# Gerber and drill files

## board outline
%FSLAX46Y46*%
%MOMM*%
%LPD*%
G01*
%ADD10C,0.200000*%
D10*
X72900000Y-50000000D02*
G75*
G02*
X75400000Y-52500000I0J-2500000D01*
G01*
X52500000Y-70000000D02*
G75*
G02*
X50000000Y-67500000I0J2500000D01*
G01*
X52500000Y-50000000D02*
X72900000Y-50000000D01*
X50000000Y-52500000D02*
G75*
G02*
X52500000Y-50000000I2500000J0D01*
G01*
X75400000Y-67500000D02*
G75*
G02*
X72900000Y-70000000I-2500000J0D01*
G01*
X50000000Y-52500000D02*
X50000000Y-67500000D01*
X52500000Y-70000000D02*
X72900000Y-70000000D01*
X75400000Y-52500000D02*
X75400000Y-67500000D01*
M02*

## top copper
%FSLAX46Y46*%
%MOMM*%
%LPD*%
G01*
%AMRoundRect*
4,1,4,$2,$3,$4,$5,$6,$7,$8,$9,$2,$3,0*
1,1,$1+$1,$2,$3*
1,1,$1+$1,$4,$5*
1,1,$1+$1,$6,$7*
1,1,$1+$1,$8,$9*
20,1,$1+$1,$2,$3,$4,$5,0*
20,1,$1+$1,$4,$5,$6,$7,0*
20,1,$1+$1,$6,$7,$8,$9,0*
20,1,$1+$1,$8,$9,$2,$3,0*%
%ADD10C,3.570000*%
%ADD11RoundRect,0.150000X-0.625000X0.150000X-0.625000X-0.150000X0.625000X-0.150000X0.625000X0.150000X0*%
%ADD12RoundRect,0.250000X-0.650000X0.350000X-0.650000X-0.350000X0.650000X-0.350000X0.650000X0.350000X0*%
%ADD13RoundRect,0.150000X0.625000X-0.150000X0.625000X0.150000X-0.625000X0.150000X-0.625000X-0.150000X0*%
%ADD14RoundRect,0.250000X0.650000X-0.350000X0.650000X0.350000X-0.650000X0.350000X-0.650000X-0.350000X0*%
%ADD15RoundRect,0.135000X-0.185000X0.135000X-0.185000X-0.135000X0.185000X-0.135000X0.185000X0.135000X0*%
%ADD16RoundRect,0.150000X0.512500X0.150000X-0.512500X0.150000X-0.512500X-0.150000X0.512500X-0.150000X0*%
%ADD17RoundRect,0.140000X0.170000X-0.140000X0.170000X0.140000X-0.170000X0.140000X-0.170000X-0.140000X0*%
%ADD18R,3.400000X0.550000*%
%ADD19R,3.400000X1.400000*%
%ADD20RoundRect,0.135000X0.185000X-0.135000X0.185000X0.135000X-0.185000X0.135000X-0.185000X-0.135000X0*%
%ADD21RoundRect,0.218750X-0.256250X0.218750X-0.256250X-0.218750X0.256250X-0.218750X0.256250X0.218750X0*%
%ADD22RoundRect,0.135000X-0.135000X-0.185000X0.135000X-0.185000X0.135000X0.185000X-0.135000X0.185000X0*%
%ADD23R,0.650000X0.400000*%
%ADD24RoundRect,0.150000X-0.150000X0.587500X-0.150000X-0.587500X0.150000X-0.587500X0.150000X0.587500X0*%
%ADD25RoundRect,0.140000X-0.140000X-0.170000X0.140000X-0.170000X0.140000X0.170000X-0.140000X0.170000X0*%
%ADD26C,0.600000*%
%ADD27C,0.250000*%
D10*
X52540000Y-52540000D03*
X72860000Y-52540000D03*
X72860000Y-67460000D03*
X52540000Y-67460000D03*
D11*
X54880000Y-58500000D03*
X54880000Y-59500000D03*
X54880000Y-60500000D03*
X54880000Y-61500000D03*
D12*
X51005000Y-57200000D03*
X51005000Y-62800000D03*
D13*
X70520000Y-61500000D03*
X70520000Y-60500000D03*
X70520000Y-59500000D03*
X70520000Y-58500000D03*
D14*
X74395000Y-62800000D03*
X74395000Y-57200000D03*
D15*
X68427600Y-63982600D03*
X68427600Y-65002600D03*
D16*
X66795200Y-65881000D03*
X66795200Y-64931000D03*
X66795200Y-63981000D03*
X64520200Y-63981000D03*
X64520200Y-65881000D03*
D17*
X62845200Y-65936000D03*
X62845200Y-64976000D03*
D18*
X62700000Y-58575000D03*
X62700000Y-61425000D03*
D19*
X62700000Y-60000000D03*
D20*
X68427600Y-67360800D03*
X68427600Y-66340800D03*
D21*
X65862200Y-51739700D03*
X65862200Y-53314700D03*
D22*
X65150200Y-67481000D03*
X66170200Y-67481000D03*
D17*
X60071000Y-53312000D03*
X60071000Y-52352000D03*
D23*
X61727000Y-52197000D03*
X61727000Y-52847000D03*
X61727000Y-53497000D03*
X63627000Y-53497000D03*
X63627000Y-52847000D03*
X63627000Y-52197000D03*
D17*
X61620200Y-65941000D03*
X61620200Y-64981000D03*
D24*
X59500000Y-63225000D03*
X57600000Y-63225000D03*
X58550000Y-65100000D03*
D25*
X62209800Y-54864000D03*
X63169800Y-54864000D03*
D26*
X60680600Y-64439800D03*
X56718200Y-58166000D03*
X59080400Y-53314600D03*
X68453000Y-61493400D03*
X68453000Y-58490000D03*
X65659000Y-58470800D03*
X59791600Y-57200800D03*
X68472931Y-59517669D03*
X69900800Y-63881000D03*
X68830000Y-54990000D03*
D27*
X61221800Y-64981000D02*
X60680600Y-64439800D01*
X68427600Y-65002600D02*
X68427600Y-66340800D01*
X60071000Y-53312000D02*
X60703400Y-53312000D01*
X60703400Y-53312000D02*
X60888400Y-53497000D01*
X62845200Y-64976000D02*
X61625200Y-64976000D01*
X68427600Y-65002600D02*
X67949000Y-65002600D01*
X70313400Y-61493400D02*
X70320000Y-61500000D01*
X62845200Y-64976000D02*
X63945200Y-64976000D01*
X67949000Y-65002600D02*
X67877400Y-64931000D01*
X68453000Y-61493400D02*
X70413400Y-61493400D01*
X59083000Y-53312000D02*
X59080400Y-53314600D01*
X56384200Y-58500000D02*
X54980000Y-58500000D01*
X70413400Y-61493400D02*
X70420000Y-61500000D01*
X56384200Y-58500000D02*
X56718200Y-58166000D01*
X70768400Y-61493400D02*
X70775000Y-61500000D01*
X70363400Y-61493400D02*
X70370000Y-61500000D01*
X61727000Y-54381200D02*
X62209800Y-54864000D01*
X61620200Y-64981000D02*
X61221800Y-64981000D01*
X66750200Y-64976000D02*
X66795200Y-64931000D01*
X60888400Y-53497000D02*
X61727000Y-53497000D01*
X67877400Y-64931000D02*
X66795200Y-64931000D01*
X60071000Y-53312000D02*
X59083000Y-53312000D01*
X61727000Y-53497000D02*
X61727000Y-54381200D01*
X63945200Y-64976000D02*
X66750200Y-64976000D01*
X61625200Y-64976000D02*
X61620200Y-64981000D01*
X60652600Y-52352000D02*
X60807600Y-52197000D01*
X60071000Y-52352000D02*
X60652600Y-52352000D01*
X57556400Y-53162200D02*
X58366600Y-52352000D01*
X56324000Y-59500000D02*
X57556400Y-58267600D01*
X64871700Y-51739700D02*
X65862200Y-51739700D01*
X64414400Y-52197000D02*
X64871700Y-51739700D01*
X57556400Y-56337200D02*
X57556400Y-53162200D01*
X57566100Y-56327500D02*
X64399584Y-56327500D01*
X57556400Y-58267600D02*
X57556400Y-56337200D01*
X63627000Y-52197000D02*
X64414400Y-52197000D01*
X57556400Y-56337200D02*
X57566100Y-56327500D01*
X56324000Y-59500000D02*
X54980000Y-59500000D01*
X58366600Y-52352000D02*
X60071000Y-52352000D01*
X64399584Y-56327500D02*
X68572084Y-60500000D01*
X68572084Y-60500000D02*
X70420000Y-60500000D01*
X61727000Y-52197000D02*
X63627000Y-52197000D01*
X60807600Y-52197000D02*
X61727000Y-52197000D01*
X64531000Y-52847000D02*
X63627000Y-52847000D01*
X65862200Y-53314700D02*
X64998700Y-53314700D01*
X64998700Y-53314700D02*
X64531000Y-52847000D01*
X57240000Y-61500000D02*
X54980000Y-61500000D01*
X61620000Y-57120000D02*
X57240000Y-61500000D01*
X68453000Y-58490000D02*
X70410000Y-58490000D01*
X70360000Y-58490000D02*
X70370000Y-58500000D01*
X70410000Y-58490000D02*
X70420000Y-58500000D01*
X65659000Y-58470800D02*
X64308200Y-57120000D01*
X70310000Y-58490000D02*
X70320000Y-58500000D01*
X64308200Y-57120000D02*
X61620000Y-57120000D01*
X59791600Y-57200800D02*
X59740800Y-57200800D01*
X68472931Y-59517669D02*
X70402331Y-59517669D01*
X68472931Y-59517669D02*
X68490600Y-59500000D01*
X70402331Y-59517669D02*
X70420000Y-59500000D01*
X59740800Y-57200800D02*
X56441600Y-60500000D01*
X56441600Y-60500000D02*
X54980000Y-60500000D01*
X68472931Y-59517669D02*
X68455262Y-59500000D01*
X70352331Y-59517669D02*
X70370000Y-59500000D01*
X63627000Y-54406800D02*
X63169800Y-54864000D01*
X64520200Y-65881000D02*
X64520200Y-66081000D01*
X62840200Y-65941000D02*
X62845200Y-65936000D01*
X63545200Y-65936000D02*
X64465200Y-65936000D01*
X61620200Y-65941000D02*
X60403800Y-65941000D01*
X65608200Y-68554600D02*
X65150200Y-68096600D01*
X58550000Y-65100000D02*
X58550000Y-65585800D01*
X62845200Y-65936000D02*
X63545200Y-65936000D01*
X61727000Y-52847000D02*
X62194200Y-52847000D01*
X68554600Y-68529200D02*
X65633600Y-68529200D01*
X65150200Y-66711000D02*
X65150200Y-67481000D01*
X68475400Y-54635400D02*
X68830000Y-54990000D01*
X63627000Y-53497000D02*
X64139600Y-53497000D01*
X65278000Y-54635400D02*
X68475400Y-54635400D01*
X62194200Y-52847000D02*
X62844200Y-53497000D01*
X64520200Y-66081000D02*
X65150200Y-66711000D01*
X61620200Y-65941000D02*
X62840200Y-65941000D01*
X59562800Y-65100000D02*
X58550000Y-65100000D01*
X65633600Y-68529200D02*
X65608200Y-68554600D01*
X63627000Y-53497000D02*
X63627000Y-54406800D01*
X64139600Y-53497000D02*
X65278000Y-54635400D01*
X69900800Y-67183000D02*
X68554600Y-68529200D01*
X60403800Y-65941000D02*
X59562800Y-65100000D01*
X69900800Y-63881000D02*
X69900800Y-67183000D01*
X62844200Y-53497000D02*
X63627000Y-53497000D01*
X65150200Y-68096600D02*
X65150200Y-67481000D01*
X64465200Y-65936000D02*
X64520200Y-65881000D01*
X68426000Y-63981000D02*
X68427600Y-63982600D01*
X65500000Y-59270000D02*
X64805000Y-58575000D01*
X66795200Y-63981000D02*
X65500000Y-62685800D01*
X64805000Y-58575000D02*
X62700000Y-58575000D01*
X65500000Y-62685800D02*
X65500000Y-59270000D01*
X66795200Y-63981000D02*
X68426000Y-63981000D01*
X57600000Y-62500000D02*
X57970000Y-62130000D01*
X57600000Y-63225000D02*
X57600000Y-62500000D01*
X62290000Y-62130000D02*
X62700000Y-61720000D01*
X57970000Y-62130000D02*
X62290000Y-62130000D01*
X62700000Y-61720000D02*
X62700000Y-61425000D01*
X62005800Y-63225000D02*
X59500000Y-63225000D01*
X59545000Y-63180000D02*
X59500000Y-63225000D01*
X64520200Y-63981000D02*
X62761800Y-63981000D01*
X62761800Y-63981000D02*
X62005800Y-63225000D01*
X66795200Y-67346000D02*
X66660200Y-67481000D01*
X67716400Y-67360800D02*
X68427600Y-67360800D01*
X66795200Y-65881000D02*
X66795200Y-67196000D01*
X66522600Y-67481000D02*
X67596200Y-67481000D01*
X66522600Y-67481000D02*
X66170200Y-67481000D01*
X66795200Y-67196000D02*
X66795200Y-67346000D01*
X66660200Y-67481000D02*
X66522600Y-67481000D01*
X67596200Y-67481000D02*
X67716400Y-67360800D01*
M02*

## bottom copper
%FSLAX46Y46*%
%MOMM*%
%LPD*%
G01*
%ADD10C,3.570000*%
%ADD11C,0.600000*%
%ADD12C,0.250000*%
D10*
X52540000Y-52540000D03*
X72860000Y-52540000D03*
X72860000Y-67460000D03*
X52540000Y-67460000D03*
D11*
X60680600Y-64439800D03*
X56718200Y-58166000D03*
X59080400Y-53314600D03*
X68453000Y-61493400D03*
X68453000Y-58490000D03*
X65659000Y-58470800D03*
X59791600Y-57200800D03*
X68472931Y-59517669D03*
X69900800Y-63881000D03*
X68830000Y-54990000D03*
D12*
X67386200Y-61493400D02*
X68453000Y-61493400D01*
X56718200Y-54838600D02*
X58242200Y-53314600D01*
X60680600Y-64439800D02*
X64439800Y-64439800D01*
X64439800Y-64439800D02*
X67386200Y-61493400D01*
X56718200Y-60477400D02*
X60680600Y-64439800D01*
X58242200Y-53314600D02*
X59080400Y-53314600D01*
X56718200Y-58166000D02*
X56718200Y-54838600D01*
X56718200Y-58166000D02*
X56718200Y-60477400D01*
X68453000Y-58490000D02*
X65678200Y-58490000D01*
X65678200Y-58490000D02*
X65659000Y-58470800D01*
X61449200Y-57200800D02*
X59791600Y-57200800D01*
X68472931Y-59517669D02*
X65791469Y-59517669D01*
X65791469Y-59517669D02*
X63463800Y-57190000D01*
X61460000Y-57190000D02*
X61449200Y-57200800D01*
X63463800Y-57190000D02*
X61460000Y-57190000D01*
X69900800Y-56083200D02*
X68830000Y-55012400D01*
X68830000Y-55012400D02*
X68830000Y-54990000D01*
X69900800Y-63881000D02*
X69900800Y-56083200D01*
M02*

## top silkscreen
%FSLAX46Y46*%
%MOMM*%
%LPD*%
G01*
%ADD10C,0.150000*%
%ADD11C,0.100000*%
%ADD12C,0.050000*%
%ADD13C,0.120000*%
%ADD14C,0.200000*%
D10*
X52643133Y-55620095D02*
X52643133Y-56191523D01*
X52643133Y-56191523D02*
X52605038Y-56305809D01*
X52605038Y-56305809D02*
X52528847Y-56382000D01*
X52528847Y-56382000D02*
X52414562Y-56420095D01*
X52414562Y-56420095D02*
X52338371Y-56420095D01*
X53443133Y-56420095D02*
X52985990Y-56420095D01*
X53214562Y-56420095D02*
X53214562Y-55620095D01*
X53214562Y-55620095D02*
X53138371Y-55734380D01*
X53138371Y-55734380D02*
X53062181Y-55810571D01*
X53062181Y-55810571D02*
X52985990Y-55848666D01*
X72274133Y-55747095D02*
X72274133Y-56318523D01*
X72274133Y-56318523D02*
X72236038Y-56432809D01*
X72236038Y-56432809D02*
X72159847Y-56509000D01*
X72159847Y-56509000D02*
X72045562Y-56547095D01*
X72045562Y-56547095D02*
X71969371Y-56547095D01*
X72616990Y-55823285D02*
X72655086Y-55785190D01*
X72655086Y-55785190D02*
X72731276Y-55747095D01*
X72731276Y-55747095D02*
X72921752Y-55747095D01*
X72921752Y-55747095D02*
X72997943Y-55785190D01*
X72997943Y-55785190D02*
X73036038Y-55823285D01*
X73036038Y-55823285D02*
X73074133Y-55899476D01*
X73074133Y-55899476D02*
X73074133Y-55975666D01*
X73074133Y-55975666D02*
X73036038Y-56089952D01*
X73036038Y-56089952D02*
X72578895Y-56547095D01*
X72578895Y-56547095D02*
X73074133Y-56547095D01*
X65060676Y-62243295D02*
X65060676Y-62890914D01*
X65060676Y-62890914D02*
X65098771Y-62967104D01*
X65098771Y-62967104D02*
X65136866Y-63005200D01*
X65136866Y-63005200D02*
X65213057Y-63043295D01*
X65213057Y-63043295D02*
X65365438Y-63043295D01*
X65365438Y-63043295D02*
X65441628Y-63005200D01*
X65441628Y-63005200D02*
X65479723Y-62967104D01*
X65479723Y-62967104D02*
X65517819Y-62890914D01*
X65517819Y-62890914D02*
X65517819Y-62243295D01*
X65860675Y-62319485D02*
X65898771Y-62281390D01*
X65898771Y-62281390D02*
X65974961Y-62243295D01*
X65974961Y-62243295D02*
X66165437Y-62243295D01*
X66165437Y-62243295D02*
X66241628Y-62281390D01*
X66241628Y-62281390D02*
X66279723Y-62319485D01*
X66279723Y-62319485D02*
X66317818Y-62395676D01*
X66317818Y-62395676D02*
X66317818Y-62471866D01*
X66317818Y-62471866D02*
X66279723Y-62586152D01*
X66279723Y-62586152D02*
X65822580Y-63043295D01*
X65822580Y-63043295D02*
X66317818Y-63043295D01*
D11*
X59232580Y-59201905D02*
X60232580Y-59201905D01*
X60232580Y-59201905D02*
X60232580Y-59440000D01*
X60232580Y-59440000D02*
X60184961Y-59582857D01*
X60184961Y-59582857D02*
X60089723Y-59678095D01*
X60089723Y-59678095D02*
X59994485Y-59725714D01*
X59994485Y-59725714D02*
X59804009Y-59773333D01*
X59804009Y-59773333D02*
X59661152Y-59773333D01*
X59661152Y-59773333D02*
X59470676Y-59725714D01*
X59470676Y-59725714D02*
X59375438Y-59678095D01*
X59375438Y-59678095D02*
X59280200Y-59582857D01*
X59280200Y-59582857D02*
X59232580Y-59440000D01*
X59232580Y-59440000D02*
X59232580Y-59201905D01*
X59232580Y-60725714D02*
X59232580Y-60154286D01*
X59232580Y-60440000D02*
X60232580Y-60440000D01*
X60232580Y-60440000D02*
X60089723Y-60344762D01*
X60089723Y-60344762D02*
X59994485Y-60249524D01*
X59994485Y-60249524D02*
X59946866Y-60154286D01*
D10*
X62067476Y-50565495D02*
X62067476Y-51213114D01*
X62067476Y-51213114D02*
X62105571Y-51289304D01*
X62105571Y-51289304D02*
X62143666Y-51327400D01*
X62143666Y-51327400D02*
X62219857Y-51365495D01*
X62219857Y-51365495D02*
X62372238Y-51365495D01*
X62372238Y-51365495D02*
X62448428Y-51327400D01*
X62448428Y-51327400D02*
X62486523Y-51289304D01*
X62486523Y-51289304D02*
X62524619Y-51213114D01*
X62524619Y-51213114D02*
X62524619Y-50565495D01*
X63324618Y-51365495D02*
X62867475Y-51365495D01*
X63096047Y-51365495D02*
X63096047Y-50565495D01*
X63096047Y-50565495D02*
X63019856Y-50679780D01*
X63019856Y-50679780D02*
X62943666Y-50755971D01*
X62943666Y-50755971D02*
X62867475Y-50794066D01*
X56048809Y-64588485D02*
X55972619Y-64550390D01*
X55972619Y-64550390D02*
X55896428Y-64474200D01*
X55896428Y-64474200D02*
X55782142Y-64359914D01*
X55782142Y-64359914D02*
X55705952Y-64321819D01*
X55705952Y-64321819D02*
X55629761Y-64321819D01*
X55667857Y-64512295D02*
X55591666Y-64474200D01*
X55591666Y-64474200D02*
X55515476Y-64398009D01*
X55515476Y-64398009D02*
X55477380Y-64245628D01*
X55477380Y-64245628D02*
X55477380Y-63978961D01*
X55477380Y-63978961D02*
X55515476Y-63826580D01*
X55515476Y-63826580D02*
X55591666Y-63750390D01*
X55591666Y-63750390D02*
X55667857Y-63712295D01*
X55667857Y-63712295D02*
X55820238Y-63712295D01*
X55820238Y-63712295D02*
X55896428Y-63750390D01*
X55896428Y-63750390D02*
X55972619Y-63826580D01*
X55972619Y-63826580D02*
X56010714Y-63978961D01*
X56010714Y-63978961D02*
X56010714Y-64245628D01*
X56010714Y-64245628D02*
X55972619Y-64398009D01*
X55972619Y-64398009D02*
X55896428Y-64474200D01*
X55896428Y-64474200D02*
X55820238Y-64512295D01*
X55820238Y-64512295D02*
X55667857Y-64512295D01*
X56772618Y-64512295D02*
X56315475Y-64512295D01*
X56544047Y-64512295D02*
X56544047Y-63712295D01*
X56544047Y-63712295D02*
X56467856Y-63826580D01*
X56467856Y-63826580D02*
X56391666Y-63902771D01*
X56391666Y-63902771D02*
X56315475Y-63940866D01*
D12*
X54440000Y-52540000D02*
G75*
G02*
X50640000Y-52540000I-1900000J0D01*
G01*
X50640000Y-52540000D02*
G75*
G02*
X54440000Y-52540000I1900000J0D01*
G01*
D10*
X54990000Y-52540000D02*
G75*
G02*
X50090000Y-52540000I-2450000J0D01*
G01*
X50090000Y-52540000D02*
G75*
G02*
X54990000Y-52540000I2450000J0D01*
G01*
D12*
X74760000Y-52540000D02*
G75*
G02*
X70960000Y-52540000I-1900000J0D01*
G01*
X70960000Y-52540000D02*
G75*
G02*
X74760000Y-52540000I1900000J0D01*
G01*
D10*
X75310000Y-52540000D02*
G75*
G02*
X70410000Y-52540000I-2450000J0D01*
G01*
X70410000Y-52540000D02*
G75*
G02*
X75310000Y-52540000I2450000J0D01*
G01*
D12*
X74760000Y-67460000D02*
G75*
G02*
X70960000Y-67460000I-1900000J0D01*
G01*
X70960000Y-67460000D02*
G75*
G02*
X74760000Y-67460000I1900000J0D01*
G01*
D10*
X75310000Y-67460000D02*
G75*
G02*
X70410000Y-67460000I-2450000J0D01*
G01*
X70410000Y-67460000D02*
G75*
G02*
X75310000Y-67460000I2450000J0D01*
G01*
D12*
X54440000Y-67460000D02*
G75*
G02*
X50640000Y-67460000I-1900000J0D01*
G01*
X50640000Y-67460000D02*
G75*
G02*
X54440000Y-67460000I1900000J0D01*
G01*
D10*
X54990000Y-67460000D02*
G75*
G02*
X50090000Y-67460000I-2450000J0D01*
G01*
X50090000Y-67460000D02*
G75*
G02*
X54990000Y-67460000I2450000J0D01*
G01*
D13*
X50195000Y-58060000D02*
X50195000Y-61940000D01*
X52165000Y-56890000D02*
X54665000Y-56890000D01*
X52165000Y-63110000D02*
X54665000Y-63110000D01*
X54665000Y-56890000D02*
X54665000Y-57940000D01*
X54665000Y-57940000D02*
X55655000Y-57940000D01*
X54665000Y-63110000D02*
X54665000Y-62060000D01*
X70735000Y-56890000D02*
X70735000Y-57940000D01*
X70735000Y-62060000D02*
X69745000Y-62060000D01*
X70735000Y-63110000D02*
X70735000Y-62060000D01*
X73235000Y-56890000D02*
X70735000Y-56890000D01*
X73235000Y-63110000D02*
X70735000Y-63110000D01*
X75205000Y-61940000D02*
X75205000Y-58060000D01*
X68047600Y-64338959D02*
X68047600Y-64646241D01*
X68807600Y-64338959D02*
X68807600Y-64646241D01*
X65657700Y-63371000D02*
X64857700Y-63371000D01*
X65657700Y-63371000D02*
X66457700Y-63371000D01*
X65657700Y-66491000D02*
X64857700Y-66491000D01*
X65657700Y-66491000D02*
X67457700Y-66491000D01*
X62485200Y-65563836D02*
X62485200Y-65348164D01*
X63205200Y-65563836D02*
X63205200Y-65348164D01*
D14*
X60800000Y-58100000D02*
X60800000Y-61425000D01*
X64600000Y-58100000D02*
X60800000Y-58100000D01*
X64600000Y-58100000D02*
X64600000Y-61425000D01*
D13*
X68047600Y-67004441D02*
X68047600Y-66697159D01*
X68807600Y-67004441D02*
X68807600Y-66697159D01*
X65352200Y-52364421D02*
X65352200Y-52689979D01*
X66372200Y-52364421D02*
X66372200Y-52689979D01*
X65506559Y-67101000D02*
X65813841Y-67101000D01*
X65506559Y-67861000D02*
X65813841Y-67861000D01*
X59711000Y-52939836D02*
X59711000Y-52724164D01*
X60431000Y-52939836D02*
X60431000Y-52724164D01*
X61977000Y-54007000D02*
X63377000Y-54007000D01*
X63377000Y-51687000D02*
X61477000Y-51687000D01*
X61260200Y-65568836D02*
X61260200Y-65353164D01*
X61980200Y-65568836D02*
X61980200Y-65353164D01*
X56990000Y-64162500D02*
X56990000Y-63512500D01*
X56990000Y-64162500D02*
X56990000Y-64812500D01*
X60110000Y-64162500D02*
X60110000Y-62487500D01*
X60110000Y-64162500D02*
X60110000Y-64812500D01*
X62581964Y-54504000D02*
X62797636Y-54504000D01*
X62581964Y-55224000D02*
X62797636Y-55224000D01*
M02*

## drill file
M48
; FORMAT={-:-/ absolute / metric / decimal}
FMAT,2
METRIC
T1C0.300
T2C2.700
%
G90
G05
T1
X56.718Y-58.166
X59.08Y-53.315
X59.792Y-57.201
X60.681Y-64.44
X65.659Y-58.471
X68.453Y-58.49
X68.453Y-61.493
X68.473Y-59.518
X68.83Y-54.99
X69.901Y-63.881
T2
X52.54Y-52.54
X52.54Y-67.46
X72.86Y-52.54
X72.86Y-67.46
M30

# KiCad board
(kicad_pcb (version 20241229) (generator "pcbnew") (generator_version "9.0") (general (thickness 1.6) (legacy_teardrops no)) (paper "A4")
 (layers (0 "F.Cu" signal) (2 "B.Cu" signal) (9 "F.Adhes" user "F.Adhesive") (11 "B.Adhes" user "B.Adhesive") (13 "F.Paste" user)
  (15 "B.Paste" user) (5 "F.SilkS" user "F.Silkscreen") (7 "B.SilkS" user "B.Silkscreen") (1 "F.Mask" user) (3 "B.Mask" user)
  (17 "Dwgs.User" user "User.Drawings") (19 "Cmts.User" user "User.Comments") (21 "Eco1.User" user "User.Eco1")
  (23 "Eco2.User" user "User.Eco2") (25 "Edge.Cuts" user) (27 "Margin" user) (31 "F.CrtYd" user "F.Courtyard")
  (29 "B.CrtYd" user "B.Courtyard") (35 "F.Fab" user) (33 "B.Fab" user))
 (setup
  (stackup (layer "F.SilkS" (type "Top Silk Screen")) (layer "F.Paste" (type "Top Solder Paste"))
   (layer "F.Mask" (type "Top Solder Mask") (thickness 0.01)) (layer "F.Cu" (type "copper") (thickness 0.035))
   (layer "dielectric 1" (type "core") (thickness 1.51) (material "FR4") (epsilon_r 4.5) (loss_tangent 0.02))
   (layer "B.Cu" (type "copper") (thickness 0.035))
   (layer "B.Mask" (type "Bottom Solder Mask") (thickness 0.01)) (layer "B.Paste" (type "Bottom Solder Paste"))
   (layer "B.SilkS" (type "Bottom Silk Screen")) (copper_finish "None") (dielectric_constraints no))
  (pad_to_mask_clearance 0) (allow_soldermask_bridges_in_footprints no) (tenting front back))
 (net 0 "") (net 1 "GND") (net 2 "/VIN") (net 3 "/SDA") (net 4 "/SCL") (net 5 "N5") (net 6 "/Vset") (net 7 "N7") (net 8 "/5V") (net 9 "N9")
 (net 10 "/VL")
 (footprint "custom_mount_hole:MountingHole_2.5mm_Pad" (layer "F.Cu") (at 52.54 52.54)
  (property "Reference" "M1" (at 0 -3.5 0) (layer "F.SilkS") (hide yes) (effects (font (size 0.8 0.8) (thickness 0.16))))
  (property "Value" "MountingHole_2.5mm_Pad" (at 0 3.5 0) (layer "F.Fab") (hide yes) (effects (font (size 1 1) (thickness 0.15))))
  (fp_circle (center 0 0) (end 1.9 0) (stroke (width 0.05) (type solid)) (fill no) (layer "F.SilkS"))
  (fp_circle (center 0 0) (end 2.45 0) (stroke (width 0.15) (type solid)) (fill no) (layer "F.SilkS"))
  (pad "~" thru_hole circle (at 0 0) (size 3.57 3.57) (drill 2.7) (layers "*.Cu" "*.Mask") (remove_unused_layers no)))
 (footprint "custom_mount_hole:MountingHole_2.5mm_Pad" (layer "F.Cu") (at 72.86 52.54)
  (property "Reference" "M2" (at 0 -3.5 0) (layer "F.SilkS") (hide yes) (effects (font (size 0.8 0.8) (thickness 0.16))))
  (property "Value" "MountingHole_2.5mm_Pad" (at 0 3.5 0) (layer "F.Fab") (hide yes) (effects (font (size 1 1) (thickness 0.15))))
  (fp_circle (center 0 0) (end 1.9 0) (stroke (width 0.05) (type solid)) (fill no) (layer "F.SilkS"))
  (fp_circle (center 0 0) (end 2.45 0) (stroke (width 0.15) (type solid)) (fill no) (layer "F.SilkS"))
  (pad "~" thru_hole circle (at 0 0) (size 3.57 3.57) (drill 2.7) (layers "*.Cu" "*.Mask") (remove_unused_layers no)))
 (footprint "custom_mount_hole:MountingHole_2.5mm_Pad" (layer "F.Cu") (at 72.86 67.46)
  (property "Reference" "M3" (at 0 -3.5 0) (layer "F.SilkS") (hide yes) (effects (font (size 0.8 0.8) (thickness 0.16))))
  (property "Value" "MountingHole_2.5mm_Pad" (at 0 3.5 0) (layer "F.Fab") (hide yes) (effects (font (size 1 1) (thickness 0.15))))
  (fp_circle (center 0 0) (end 1.9 0) (stroke (width 0.05) (type solid)) (fill no) (layer "F.SilkS"))
  (fp_circle (center 0 0) (end 2.45 0) (stroke (width 0.15) (type solid)) (fill no) (layer "F.SilkS"))
  (pad "~" thru_hole circle (at 0 0) (size 3.57 3.57) (drill 2.7) (layers "*.Cu" "*.Mask") (remove_unused_layers no)))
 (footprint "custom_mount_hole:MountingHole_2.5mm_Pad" (layer "F.Cu") (at 52.54 67.46)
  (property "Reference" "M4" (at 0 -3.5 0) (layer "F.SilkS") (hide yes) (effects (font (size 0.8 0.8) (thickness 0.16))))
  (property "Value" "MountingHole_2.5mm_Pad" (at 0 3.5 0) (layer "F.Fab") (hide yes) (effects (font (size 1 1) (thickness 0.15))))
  (fp_circle (center 0 0) (end 1.9 0) (stroke (width 0.05) (type solid)) (fill no) (layer "F.SilkS"))
  (fp_circle (center 0 0) (end 2.45 0) (stroke (width 0.15) (type solid)) (fill no) (layer "F.SilkS"))
  (pad "~" thru_hole circle (at 0 0) (size 3.57 3.57) (drill 2.7) (layers "*.Cu" "*.Mask") (remove_unused_layers no)))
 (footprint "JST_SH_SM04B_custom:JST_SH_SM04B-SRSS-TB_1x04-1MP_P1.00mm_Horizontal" (layer "F.Cu") (at 52.88 60 -90)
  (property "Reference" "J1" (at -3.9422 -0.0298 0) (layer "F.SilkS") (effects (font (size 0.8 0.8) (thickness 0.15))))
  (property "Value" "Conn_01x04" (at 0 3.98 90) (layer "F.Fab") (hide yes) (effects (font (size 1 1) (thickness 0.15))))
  (fp_line (start -1.94 2.685) (end 1.94 2.685) (stroke (width 0.12) (type solid)) (layer "F.SilkS"))
  (fp_line (start -3.11 0.715) (end -3.11 -1.785) (stroke (width 0.12) (type solid)) (layer "F.SilkS"))
  (fp_line (start 3.11 0.715) (end 3.11 -1.785) (stroke (width 0.12) (type solid)) (layer "F.SilkS"))
  (fp_line (start -3.11 -1.785) (end -2.06 -1.785) (stroke (width 0.12) (type solid)) (layer "F.SilkS"))
  (fp_line (start -2.06 -1.785) (end -2.06 -2.775) (stroke (width 0.12) (type solid)) (layer "F.SilkS"))
  (fp_line (start 3.11 -1.785) (end 2.06 -1.785) (stroke (width 0.12) (type solid)) (layer "F.SilkS"))
  (pad "1" smd roundrect (at -1.5 -2 270) (size 0.6 1.55) (layers "F.Cu" "F.Mask" "F.Paste") (roundrect_rratio 0.25) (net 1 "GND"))
  (pad "2" smd roundrect (at -0.5 -2 270) (size 0.6 1.55) (layers "F.Cu" "F.Mask" "F.Paste") (roundrect_rratio 0.25) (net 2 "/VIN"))
  (pad "3" smd roundrect (at 0.5 -2 270) (size 0.6 1.55) (layers "F.Cu" "F.Mask" "F.Paste") (roundrect_rratio 0.25) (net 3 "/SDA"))
  (pad "4" smd roundrect (at 1.5 -2 270) (size 0.6 1.55) (layers "F.Cu" "F.Mask" "F.Paste") (roundrect_rratio 0.25) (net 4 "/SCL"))
  (pad "MP" smd roundrect (at -2.8 1.875 270) (size 1.2 1.8) (layers "F.Cu" "F.Mask" "F.Paste") (roundrect_rratio 0.2083333333))
  (pad "MP" smd roundrect (at 2.8 1.875 270) (size 1.2 1.8) (layers "F.Cu" "F.Mask" "F.Paste") (roundrect_rratio 0.2083333333)))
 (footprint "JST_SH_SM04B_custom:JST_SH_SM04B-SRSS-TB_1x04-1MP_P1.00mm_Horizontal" (layer "F.Cu") (at 72.52 60 90)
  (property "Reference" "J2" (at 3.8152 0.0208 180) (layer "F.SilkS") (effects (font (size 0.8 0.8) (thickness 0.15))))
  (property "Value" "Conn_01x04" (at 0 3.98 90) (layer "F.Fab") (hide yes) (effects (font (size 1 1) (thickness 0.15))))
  (fp_line (start 3.11 -1.785) (end 2.06 -1.785) (stroke (width 0.12) (type solid)) (layer "F.SilkS"))
  (fp_line (start -2.06 -1.785) (end -2.06 -2.775) (stroke (width 0.12) (type solid)) (layer "F.SilkS"))
  (fp_line (start -3.11 -1.785) (end -2.06 -1.785) (stroke (width 0.12) (type solid)) (layer "F.SilkS"))
  (fp_line (start 3.11 0.715) (end 3.11 -1.785) (stroke (width 0.12) (type solid)) (layer "F.SilkS"))
  (fp_line (start -3.11 0.715) (end -3.11 -1.785) (stroke (width 0.12) (type solid)) (layer "F.SilkS"))
  (fp_line (start -1.94 2.685) (end 1.94 2.685) (stroke (width 0.12) (type solid)) (layer "F.SilkS"))
  (pad "1" smd roundrect (at -1.5 -2 90) (size 0.6 1.55) (layers "F.Cu" "F.Mask" "F.Paste") (roundrect_rratio 0.25) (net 1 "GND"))
  (pad "2" smd roundrect (at -0.5 -2 90) (size 0.6 1.55) (layers "F.Cu" "F.Mask" "F.Paste") (roundrect_rratio 0.25) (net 2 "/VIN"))
  (pad "3" smd roundrect (at 0.5 -2 90) (size 0.6 1.55) (layers "F.Cu" "F.Mask" "F.Paste") (roundrect_rratio 0.25) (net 3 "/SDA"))
  (pad "4" smd roundrect (at 1.5 -2 90) (size 0.6 1.55) (layers "F.Cu" "F.Mask" "F.Paste") (roundrect_rratio 0.25) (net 4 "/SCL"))
  (pad "MP" smd roundrect (at -2.8 1.875 90) (size 1.2 1.8) (layers "F.Cu" "F.Mask" "F.Paste") (roundrect_rratio 0.2083333333))
  (pad "MP" smd roundrect (at 2.8 1.875 90) (size 1.2 1.8) (layers "F.Cu" "F.Mask" "F.Paste") (roundrect_rratio 0.2083333333)))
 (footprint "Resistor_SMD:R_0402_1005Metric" (layer "F.Cu") (at 68.4276 64.4926 -90)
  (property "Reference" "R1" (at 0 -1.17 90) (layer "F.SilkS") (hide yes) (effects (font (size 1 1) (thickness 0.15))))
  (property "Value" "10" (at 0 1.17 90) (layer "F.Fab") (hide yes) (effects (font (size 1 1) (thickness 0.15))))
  (fp_line (start -0.153641 0.38) (end 0.153641 0.38) (stroke (width 0.12) (type solid)) (layer "F.SilkS"))
  (fp_line (start -0.153641 -0.38) (end 0.153641 -0.38) (stroke (width 0.12) (type solid)) (layer "F.SilkS"))
  (pad "1" smd roundrect (at -0.51 0 270) (size 0.54 0.64) (layers "F.Cu" "F.Mask" "F.Paste") (roundrect_rratio 0.25) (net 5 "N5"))
  (pad "2" smd roundrect (at 0.51 0 270) (size 0.54 0.64) (layers "F.Cu" "F.Mask" "F.Paste") (roundrect_rratio 0.25) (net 1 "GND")))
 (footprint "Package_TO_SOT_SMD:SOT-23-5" (layer "F.Cu") (at 65.6577 64.931 180)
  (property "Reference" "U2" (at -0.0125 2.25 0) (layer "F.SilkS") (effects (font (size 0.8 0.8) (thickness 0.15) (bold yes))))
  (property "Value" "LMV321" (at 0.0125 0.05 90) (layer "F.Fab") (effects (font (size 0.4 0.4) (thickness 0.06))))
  (fp_line (start 0 1.56) (end 0.8 1.56) (stroke (width 0.12) (type solid)) (layer "F.SilkS"))
  (fp_line (start 0 1.56) (end -0.8 1.56) (stroke (width 0.12) (type solid)) (layer "F.SilkS"))
  (fp_line (start 0 -1.56) (end 0.8 -1.56) (stroke (width 0.12) (type solid)) (layer "F.SilkS"))
  (fp_line (start 0 -1.56) (end -1.8 -1.56) (stroke (width 0.12) (type solid)) (layer "F.SilkS"))
  (pad "1" smd roundrect (at -1.1375 -0.95 180) (size 1.325 0.6) (layers "F.Cu" "F.Mask" "F.Paste") (roundrect_rratio 0.25) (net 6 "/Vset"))
  (pad "2" smd roundrect (at -1.1375 0 180) (size 1.325 0.6) (layers "F.Cu" "F.Mask" "F.Paste") (roundrect_rratio 0.25) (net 1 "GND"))
  (pad "3" smd roundrect (at -1.1375 0.95 180) (size 1.325 0.6) (layers "F.Cu" "F.Mask" "F.Paste") (roundrect_rratio 0.25) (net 5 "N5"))
  (pad "4" smd roundrect (at 1.1375 0.95 180) (size 1.325 0.6) (layers "F.Cu" "F.Mask" "F.Paste") (roundrect_rratio 0.25) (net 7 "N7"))
  (pad "5" smd roundrect (at 1.1375 -0.95 180) (size 1.325 0.6) (layers "F.Cu" "F.Mask" "F.Paste") (roundrect_rratio 0.25) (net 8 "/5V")))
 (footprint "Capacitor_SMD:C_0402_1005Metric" (layer "F.Cu") (at 62.8452 65.456 90)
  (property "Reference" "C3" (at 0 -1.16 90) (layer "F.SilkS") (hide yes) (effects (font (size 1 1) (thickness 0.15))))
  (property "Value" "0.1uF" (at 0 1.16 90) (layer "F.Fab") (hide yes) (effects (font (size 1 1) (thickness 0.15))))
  (fp_line (start -0.107836 -0.36) (end 0.107836 -0.36) (stroke (width 0.12) (type solid)) (layer "F.SilkS"))
  (fp_line (start -0.107836 0.36) (end 0.107836 0.36) (stroke (width 0.12) (type solid)) (layer "F.SilkS"))
  (pad "1" smd roundrect (at -0.48 0 90) (size 0.56 0.62) (layers "F.Cu" "F.Mask" "F.Paste") (roundrect_rratio 0.25) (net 8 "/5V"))
  (pad "2" smd roundrect (at 0.48 0 90) (size 0.56 0.62) (layers "F.Cu" "F.Mask" "F.Paste") (roundrect_rratio 0.25) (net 1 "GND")))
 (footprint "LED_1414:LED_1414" (layer "F.Cu") (at 62.7 60 -90)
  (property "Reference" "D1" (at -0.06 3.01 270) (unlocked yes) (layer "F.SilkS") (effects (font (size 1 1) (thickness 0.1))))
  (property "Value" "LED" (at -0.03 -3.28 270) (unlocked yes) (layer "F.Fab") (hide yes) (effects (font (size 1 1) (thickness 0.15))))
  (fp_line (start -1.9 1.9) (end 1.425 1.9) (stroke (width 0.2) (type default)) (layer "F.SilkS"))
  (fp_line (start -1.9 -1.9) (end -1.9 1.9) (stroke (width 0.2) (type default)) (layer "F.SilkS"))
  (fp_line (start -1.9 -1.9) (end 1.425 -1.9) (stroke (width 0.2) (type default)) (layer "F.SilkS"))
  (pad "1" smd rect (at -1.425 0 270) (size 0.55 3.4) (layers "F.Cu" "F.Mask" "F.Paste") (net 5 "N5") (thermal_bridge_angle 45))
  (pad "2" smd rect (at 1.425 0 270) (size 0.55 3.4) (layers "F.Cu" "F.Mask" "F.Paste") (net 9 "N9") (thermal_bridge_angle 45))
  (pad "3" smd rect (at 0 0 270) (size 1.4 3.4) (layers "F.Cu" "F.Mask" "F.Paste") (thermal_bridge_angle 45)))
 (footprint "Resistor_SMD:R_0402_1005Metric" (layer "F.Cu") (at 68.4276 66.8508 90)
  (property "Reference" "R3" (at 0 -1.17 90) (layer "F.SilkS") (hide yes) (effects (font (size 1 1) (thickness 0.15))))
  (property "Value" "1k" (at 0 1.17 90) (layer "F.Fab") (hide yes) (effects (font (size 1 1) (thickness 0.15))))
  (fp_line (start -0.153641 -0.38) (end 0.153641 -0.38) (stroke (width 0.12) (type solid)) (layer "F.SilkS"))
  (fp_line (start -0.153641 0.38) (end 0.153641 0.38) (stroke (width 0.12) (type solid)) (layer "F.SilkS"))
  (pad "1" smd roundrect (at -0.51 0 90) (size 0.54 0.64) (layers "F.Cu" "F.Mask" "F.Paste") (roundrect_rratio 0.25) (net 6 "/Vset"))
  (pad "2" smd roundrect (at 0.51 0 90) (size 0.54 0.64) (layers "F.Cu" "F.Mask" "F.Paste") (roundrect_rratio 0.25) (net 1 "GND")))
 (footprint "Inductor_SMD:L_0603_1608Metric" (layer "F.Cu") (at 65.8622 52.5272 -90)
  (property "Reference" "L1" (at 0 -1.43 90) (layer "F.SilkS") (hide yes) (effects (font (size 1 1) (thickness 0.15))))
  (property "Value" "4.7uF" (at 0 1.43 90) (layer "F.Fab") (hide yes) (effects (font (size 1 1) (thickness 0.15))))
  (fp_line (start -0.162779 0.51) (end 0.162779 0.51) (stroke (width 0.12) (type solid)) (layer "F.SilkS"))
  (fp_line (start -0.162779 -0.51) (end 0.162779 -0.51) (stroke (width 0.12) (type solid)) (layer "F.SilkS"))
  (pad "1" smd roundrect (at -0.7875 0 270) (size 0.875 0.95) (layers "F.Cu" "F.Mask" "F.Paste") (roundrect_rratio 0.25) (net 2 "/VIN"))
  (pad "2" smd roundrect (at 0.7875 0 270) (size 0.875 0.95) (layers "F.Cu" "F.Mask" "F.Paste") (roundrect_rratio 0.25) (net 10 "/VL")))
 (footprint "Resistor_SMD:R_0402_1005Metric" (layer "F.Cu") (at 65.6602 67.481)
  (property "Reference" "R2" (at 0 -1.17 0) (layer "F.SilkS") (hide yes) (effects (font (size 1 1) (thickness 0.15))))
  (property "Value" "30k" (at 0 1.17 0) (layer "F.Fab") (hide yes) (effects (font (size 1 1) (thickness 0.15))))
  (fp_line (start -0.153641 -0.38) (end 0.153641 -0.38) (stroke (width 0.12) (type solid)) (layer "F.SilkS"))
  (fp_line (start -0.153641 0.38) (end 0.153641 0.38) (stroke (width 0.12) (type solid)) (layer "F.SilkS"))
  (pad "1" smd roundrect (at -0.51 0) (size 0.54 0.64) (layers "F.Cu" "F.Mask" "F.Paste") (roundrect_rratio 0.25) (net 8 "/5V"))
  (pad "2" smd roundrect (at 0.51 0) (size 0.54 0.64) (layers "F.Cu" "F.Mask" "F.Paste") (roundrect_rratio 0.25) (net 6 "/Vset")))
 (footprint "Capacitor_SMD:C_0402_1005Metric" (layer "F.Cu") (at 60.071 52.832 90)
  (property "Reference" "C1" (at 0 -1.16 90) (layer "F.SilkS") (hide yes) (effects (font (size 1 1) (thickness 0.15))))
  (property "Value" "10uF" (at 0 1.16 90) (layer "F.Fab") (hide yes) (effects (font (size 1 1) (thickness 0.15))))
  (fp_line (start -0.107836 -0.36) (end 0.107836 -0.36) (stroke (width 0.12) (type solid)) (layer "F.SilkS"))
  (fp_line (start -0.107836 0.36) (end 0.107836 0.36) (stroke (width 0.12) (type solid)) (layer "F.SilkS"))
  (pad "1" smd roundrect (at -0.48 0 90) (size 0.56 0.62) (layers "F.Cu" "F.Mask" "F.Paste") (roundrect_rratio 0.25) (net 1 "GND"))
  (pad "2" smd roundrect (at 0.48 0 90) (size 0.56 0.62) (layers "F.Cu" "F.Mask" "F.Paste") (roundrect_rratio 0.25) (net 2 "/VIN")))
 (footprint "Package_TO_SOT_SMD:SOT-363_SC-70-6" (layer "F.Cu") (at 62.677 52.847)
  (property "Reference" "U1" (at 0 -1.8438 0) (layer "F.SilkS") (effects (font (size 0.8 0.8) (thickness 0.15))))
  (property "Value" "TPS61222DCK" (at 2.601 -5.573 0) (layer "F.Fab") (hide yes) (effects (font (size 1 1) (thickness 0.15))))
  (fp_line (start -0.7 1.16) (end 0.7 1.16) (stroke (width 0.12) (type solid)) (layer "F.SilkS"))
  (fp_line (start 0.7 -1.16) (end -1.2 -1.16) (stroke (width 0.12) (type solid)) (layer "F.SilkS"))
  (pad "1" smd rect (at -0.95 -0.65) (size 0.65 0.4) (layers "F.Cu" "F.Mask" "F.Paste") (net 2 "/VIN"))
  (pad "2" smd rect (at -0.95 0) (size 0.65 0.4) (layers "F.Cu" "F.Mask" "F.Paste") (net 8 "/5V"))
  (pad "3" smd rect (at -0.95 0.65) (size 0.65 0.4) (layers "F.Cu" "F.Mask" "F.Paste") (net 1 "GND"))
  (pad "4" smd rect (at 0.95 0.65) (size 0.65 0.4) (layers "F.Cu" "F.Mask" "F.Paste") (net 8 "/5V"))
  (pad "5" smd rect (at 0.95 0) (size 0.65 0.4) (layers "F.Cu" "F.Mask" "F.Paste") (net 10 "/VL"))
  (pad "6" smd rect (at 0.95 -0.65) (size 0.65 0.4) (layers "F.Cu" "F.Mask" "F.Paste") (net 2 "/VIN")))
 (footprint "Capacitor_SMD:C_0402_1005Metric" (layer "F.Cu") (at 61.6202 65.461 90)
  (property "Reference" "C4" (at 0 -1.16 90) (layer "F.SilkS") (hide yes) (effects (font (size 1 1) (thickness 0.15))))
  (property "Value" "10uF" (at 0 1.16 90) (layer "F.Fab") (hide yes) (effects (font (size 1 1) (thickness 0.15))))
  (fp_line (start -0.107836 -0.36) (end 0.107836 -0.36) (stroke (width 0.12) (type solid)) (layer "F.SilkS"))
  (fp_line (start -0.107836 0.36) (end 0.107836 0.36) (stroke (width 0.12) (type solid)) (layer "F.SilkS"))
  (pad "1" smd roundrect (at -0.48 0 90) (size 0.56 0.62) (layers "F.Cu" "F.Mask" "F.Paste") (roundrect_rratio 0.25) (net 8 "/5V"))
  (pad "2" smd roundrect (at 0.48 0 90) (size 0.56 0.62) (layers "F.Cu" "F.Mask" "F.Paste") (roundrect_rratio 0.25) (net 1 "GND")))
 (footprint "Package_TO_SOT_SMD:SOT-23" (layer "F.Cu") (at 58.55 64.1625 -90)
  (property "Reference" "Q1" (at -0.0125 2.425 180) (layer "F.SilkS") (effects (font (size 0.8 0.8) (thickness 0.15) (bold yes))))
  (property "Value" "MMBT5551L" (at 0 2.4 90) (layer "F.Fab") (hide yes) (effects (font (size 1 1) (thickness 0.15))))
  (fp_line (start 0 1.56) (end -0.65 1.56) (stroke (width 0.12) (type solid)) (layer "F.SilkS"))
  (fp_line (start 0 1.56) (end 0.65 1.56) (stroke (width 0.12) (type solid)) (layer "F.SilkS"))
  (fp_line (start 0 -1.56) (end -1.675 -1.56) (stroke (width 0.12) (type solid)) (layer "F.SilkS"))
  (fp_line (start 0 -1.56) (end 0.65 -1.56) (stroke (width 0.12) (type solid)) (layer "F.SilkS"))
  (pad "1" smd roundrect (at -0.9375 -0.95 270) (size 1.475 0.6) (layers "F.Cu" "F.Mask" "F.Paste") (roundrect_rratio 0.25) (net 7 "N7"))
  (pad "2" smd roundrect (at -0.9375 0.95 270) (size 1.475 0.6) (layers "F.Cu" "F.Mask" "F.Paste") (roundrect_rratio 0.25) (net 9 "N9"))
  (pad "3" smd roundrect (at 0.9375 0 270) (size 1.475 0.6) (layers "F.Cu" "F.Mask" "F.Paste") (roundrect_rratio 0.25) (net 8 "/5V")))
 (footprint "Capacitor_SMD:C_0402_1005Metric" (layer "F.Cu") (at 62.6898 54.864)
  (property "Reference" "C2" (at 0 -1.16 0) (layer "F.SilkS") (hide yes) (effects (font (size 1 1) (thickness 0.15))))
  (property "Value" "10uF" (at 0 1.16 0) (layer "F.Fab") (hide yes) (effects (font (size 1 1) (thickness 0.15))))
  (fp_line (start -0.107836 -0.36) (end 0.107836 -0.36) (stroke (width 0.12) (type solid)) (layer "F.SilkS"))
  (fp_line (start -0.107836 0.36) (end 0.107836 0.36) (stroke (width 0.12) (type solid)) (layer "F.SilkS"))
  (pad "1" smd roundrect (at -0.48 0) (size 0.56 0.62) (layers "F.Cu" "F.Mask" "F.Paste") (roundrect_rratio 0.25) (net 1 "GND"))
  (pad "2" smd roundrect (at 0.48 0) (size 0.56 0.62) (layers "F.Cu" "F.Mask" "F.Paste") (roundrect_rratio 0.25) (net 8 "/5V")))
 (gr_arc (start 72.9 50) (mid 74.667767 50.732233) (end 75.4 52.5) (stroke (width 0.2) (type solid)) (layer "Edge.Cuts"))
 (gr_arc (start 52.5 70) (mid 50.732233 69.267767) (end 50 67.5) (stroke (width 0.2) (type solid)) (layer "Edge.Cuts"))
 (gr_line (start 52.5 50) (end 72.9 50) (stroke (width 0.2) (type solid)) (layer "Edge.Cuts"))
 (gr_arc (start 50 52.5) (mid 50.732233 50.732233) (end 52.5 50) (stroke (width 0.2) (type solid)) (layer "Edge.Cuts"))
 (gr_arc (start 75.4 67.5) (mid 74.667767 69.267767) (end 72.9 70) (stroke (width 0.2) (type solid)) (layer "Edge.Cuts"))
 (gr_line (start 50 52.5) (end 50 67.5) (stroke (width 0.2) (type solid)) (layer "Edge.Cuts"))
 (gr_line (start 52.5 70) (end 72.9 70) (stroke (width 0.2) (type solid)) (layer "Edge.Cuts"))
 (gr_line (start 75.4 52.5) (end 75.4 67.5) (stroke (width 0.2) (type solid)) (layer "Edge.Cuts"))
 (segment (start 61.2218 64.981) (end 60.6806 64.4398) (width 0.25) (layer "F.Cu") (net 1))
 (segment (start 68.4276 65.0026) (end 68.4276 66.3408) (width 0.25) (layer "F.Cu") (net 1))
 (segment (start 60.071 53.312) (end 60.7034 53.312) (width 0.25) (layer "F.Cu") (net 1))
 (segment (start 60.7034 53.312) (end 60.8884 53.497) (width 0.25) (layer "F.Cu") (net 1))
 (segment (start 62.8452 64.976) (end 61.6252 64.976) (width 0.25) (layer "F.Cu") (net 1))
 (segment (start 68.4276 65.0026) (end 67.949 65.0026) (width 0.25) (layer "F.Cu") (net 1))
 (segment (start 70.3134 61.4934) (end 70.32 61.5) (width 0.25) (layer "F.Cu") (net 1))
 (segment (start 62.8452 64.976) (end 63.9452 64.976) (width 0.25) (layer "F.Cu") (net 1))
 (segment (start 67.949 65.0026) (end 67.8774 64.931) (width 0.25) (layer "F.Cu") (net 1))
 (segment (start 68.453 61.4934) (end 70.4134 61.4934) (width 0.25) (layer "F.Cu") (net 1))
 (segment (start 59.083 53.312) (end 59.0804 53.3146) (width 0.25) (layer "F.Cu") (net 1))
 (segment (start 56.3842 58.5) (end 54.98 58.5) (width 0.25) (layer "F.Cu") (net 1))
 (segment (start 70.4134 61.4934) (end 70.42 61.5) (width 0.25) (layer "F.Cu") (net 1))
 (segment (start 56.3842 58.5) (end 56.7182 58.166) (width 0.25) (layer "F.Cu") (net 1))
 (segment (start 70.7684 61.4934) (end 70.775 61.5) (width 0.25) (layer "F.Cu") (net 1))
 (segment (start 70.3634 61.4934) (end 70.37 61.5) (width 0.25) (layer "F.Cu") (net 1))
 (segment (start 61.727 54.3812) (end 62.2098 54.864) (width 0.25) (layer "F.Cu") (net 1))
 (segment (start 61.6202 64.981) (end 61.2218 64.981) (width 0.25) (layer "F.Cu") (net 1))
 (segment (start 66.7502 64.976) (end 66.7952 64.931) (width 0.25) (layer "F.Cu") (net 1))
 (segment (start 60.8884 53.497) (end 61.727 53.497) (width 0.25) (layer "F.Cu") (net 1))
 (segment (start 67.8774 64.931) (end 66.7952 64.931) (width 0.25) (layer "F.Cu") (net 1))
 (segment (start 60.071 53.312) (end 59.083 53.312) (width 0.25) (layer "F.Cu") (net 1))
 (segment (start 61.727 53.497) (end 61.727 54.3812) (width 0.25) (layer "F.Cu") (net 1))
 (segment (start 63.9452 64.976) (end 66.7502 64.976) (width 0.25) (layer "F.Cu") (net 1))
 (segment (start 61.6252 64.976) (end 61.6202 64.981) (width 0.25) (layer "F.Cu") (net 1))
 (via (at 60.6806 64.4398) (size 0.6) (drill 0.3) (layers "F.Cu" "B.Cu") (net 1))
 (via (at 56.7182 58.166) (size 0.6) (drill 0.3) (layers "F.Cu" "B.Cu") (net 1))
 (via (at 59.0804 53.3146) (size 0.6) (drill 0.3) (layers "F.Cu" "B.Cu") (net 1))
 (via (at 68.453 61.4934) (size 0.6) (drill 0.3) (layers "F.Cu" "B.Cu") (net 1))
 (segment (start 67.3862 61.4934) (end 68.453 61.4934) (width 0.25) (layer "B.Cu") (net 1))
 (segment (start 56.7182 54.8386) (end 58.2422 53.3146) (width 0.25) (layer "B.Cu") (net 1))
 (segment (start 60.6806 64.4398) (end 64.4398 64.4398) (width 0.25) (layer "B.Cu") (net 1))
 (segment (start 64.4398 64.4398) (end 67.3862 61.4934) (width 0.25) (layer "B.Cu") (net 1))
 (segment (start 56.7182 60.4774) (end 60.6806 64.4398) (width 0.25) (layer "B.Cu") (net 1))
 (segment (start 58.2422 53.3146) (end 59.0804 53.3146) (width 0.25) (layer "B.Cu") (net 1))
 (segment (start 56.7182 58.166) (end 56.7182 54.8386) (width 0.25) (layer "B.Cu") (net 1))
 (segment (start 56.7182 58.166) (end 56.7182 60.4774) (width 0.25) (layer "B.Cu") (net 1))
 (segment (start 60.6526 52.352) (end 60.8076 52.197) (width 0.25) (layer "F.Cu") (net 2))
 (segment (start 60.071 52.352) (end 60.6526 52.352) (width 0.25) (layer "F.Cu") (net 2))
 (segment (start 57.5564 53.1622) (end 58.3666 52.352) (width 0.25) (layer "F.Cu") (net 2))
 (segment (start 56.324 59.5) (end 57.5564 58.2676) (width 0.25) (layer "F.Cu") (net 2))
 (segment (start 64.8717 51.7397) (end 65.8622 51.7397) (width 0.25) (layer "F.Cu") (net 2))
 (segment (start 64.4144 52.197) (end 64.8717 51.7397) (width 0.25) (layer "F.Cu") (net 2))
 (segment (start 57.5564 56.3372) (end 57.5564 53.1622) (width 0.25) (layer "F.Cu") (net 2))
 (segment (start 57.5661 56.3275) (end 64.399584 56.3275) (width 0.25) (layer "F.Cu") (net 2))
 (segment (start 57.5564 58.2676) (end 57.5564 56.3372) (width 0.25) (layer "F.Cu") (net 2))
 (segment (start 63.627 52.197) (end 64.4144 52.197) (width 0.25) (layer "F.Cu") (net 2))
 (segment (start 57.5564 56.3372) (end 57.5661 56.3275) (width 0.25) (layer "F.Cu") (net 2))
 (segment (start 56.324 59.5) (end 54.98 59.5) (width 0.25) (layer "F.Cu") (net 2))
 (segment (start 58.3666 52.352) (end 60.071 52.352) (width 0.25) (layer "F.Cu") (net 2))
 (segment (start 64.399584 56.3275) (end 68.572084 60.5) (width 0.25) (layer "F.Cu") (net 2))
 (segment (start 68.572084 60.5) (end 70.42 60.5) (width 0.25) (layer "F.Cu") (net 2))
 (segment (start 61.727 52.197) (end 63.627 52.197) (width 0.25) (layer "F.Cu") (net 2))
 (segment (start 60.8076 52.197) (end 61.727 52.197) (width 0.25) (layer "F.Cu") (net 2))
 (segment (start 64.531 52.847) (end 63.627 52.847) (width 0.25) (layer "F.Cu") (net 10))
 (segment (start 65.8622 53.3147) (end 64.9987 53.3147) (width 0.25) (layer "F.Cu") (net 10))
 (segment (start 64.9987 53.3147) (end 64.531 52.847) (width 0.25) (layer "F.Cu") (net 10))
 (segment (start 57.24 61.5) (end 54.98 61.5) (width 0.25) (layer "F.Cu") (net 4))
 (segment (start 61.62 57.12) (end 57.24 61.5) (width 0.25) (layer "F.Cu") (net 4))
 (segment (start 68.453 58.49) (end 70.41 58.49) (width 0.25) (layer "F.Cu") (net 4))
 (segment (start 70.36 58.49) (end 70.37 58.5) (width 0.25) (layer "F.Cu") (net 4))
 (segment (start 70.41 58.49) (end 70.42 58.5) (width 0.25) (layer "F.Cu") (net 4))
 (segment (start 65.659 58.4708) (end 64.3082 57.12) (width 0.25) (layer "F.Cu") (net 4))
 (segment (start 70.31 58.49) (end 70.32 58.5) (width 0.25) (layer "F.Cu") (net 4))
 (segment (start 64.3082 57.12) (end 61.62 57.12) (width 0.25) (layer "F.Cu") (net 4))
 (via (at 68.453 58.49) (size 0.6) (drill 0.3) (layers "F.Cu" "B.Cu") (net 4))
 (via (at 65.659 58.4708) (size 0.6) (drill 0.3) (layers "F.Cu" "B.Cu") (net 4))
 (segment (start 68.453 58.49) (end 65.6782 58.49) (width 0.25) (layer "B.Cu") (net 4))
 (segment (start 65.6782 58.49) (end 65.659 58.4708) (width 0.25) (layer "B.Cu") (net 4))
 (segment (start 59.7916 57.2008) (end 59.7408 57.2008) (width 0.25) (layer "F.Cu") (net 3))
 (segment (start 68.472931 59.517669) (end 70.402331 59.517669) (width 0.25) (layer "F.Cu") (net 3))
 (segment (start 68.472931 59.517669) (end 68.4906 59.5) (width 0.25) (layer "F.Cu") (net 3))
 (segment (start 70.402331 59.517669) (end 70.42 59.5) (width 0.25) (layer "F.Cu") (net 3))
 (segment (start 59.7408 57.2008) (end 56.4416 60.5) (width 0.25) (layer "F.Cu") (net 3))
 (segment (start 56.4416 60.5) (end 54.98 60.5) (width 0.25) (layer "F.Cu") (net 3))
 (segment (start 68.472931 59.517669) (end 68.455262 59.5) (width 0.25) (layer "F.Cu") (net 3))
 (segment (start 70.352331 59.517669) (end 70.37 59.5) (width 0.25) (layer "F.Cu") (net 3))
 (via (at 59.7916 57.2008) (size 0.6) (drill 0.3) (layers "F.Cu" "B.Cu") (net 3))
 (via (at 68.472931 59.517669) (size 0.6) (drill 0.3) (layers "F.Cu" "B.Cu") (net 3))
 (segment (start 61.4492 57.2008) (end 59.7916 57.2008) (width 0.25) (layer "B.Cu") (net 3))
 (segment (start 68.472931 59.517669) (end 65.791469 59.517669) (width 0.25) (layer "B.Cu") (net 3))
 (segment (start 65.791469 59.517669) (end 63.4638 57.19) (width 0.25) (layer "B.Cu") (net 3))
 (segment (start 61.46 57.19) (end 61.4492 57.2008) (width 0.25) (layer "B.Cu") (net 3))
 (segment (start 63.4638 57.19) (end 61.46 57.19) (width 0.25) (layer "B.Cu") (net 3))
 (segment (start 63.627 54.4068) (end 63.1698 54.864) (width 0.25) (layer "F.Cu") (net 8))
 (segment (start 64.5202 65.881) (end 64.5202 66.081) (width 0.25) (layer "F.Cu") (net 8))
 (segment (start 62.8402 65.941) (end 62.8452 65.936) (width 0.25) (layer "F.Cu") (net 8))
 (segment (start 63.5452 65.936) (end 64.4652 65.936) (width 0.25) (layer "F.Cu") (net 8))
 (segment (start 61.6202 65.941) (end 60.4038 65.941) (width 0.25) (layer "F.Cu") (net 8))
 (segment (start 65.6082 68.5546) (end 65.1502 68.0966) (width 0.25) (layer "F.Cu") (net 8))
 (segment (start 58.55 65.1) (end 58.55 65.5858) (width 0.25) (layer "F.Cu") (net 8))
 (segment (start 62.8452 65.936) (end 63.5452 65.936) (width 0.25) (layer "F.Cu") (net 8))
 (segment (start 61.727 52.847) (end 62.1942 52.847) (width 0.25) (layer "F.Cu") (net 8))
 (segment (start 68.5546 68.5292) (end 65.6336 68.5292) (width 0.25) (layer "F.Cu") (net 8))
 (segment (start 65.1502 66.711) (end 65.1502 67.481) (width 0.25) (layer "F.Cu") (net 8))
 (segment (start 68.4754 54.6354) (end 68.83 54.99) (width 0.25) (layer "F.Cu") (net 8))
 (segment (start 63.627 53.497) (end 64.1396 53.497) (width 0.25) (layer "F.Cu") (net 8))
 (segment (start 65.278 54.6354) (end 68.4754 54.6354) (width 0.25) (layer "F.Cu") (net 8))
 (segment (start 62.1942 52.847) (end 62.8442 53.497) (width 0.25) (layer "F.Cu") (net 8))
 (segment (start 64.5202 66.081) (end 65.1502 66.711) (width 0.25) (layer "F.Cu") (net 8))
 (segment (start 61.6202 65.941) (end 62.8402 65.941) (width 0.25) (layer "F.Cu") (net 8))
 (segment (start 59.5628 65.1) (end 58.55 65.1) (width 0.25) (layer "F.Cu") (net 8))
 (segment (start 65.6336 68.5292) (end 65.6082 68.5546) (width 0.25) (layer "F.Cu") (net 8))
 (segment (start 63.627 53.497) (end 63.627 54.4068) (width 0.25) (layer "F.Cu") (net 8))
 (segment (start 64.1396 53.497) (end 65.278 54.6354) (width 0.25) (layer "F.Cu") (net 8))
 (segment (start 69.9008 67.183) (end 68.5546 68.5292) (width 0.25) (layer "F.Cu") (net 8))
 (segment (start 60.4038 65.941) (end 59.5628 65.1) (width 0.25) (layer "F.Cu") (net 8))
 (segment (start 69.9008 63.881) (end 69.9008 67.183) (width 0.25) (layer "F.Cu") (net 8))
 (segment (start 62.8442 53.497) (end 63.627 53.497) (width 0.25) (layer "F.Cu") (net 8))
 (segment (start 65.1502 68.0966) (end 65.1502 67.481) (width 0.25) (layer "F.Cu") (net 8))
 (segment (start 64.4652 65.936) (end 64.5202 65.881) (width 0.25) (layer "F.Cu") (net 8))
 (via (at 69.9008 63.881) (size 0.6) (drill 0.3) (layers "F.Cu" "B.Cu") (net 8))
 (via (at 68.83 54.99) (size 0.6) (drill 0.3) (layers "F.Cu" "B.Cu") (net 8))
 (segment (start 69.9008 56.0832) (end 68.83 55.0124) (width 0.25) (layer "B.Cu") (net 8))
 (segment (start 68.83 55.0124) (end 68.83 54.99) (width 0.25) (layer "B.Cu") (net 8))
 (segment (start 69.9008 63.881) (end 69.9008 56.0832) (width 0.25) (layer "B.Cu") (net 8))
 (segment (start 68.426 63.981) (end 68.4276 63.9826) (width 0.25) (layer "F.Cu") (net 5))
 (segment (start 65.5 59.27) (end 64.805 58.575) (width 0.25) (layer "F.Cu") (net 5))
 (segment (start 66.7952 63.981) (end 65.5 62.6858) (width 0.25) (layer "F.Cu") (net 5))
 (segment (start 64.805 58.575) (end 62.7 58.575) (width 0.25) (layer "F.Cu") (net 5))
 (segment (start 65.5 62.6858) (end 65.5 59.27) (width 0.25) (layer "F.Cu") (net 5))
 (segment (start 66.7952 63.981) (end 68.426 63.981) (width 0.25) (layer "F.Cu") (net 5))
 (segment (start 57.6 62.5) (end 57.97 62.13) (width 0.25) (layer "F.Cu") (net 9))
 (segment (start 57.6 63.225) (end 57.6 62.5) (width 0.25) (layer "F.Cu") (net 9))
 (segment (start 62.29 62.13) (end 62.7 61.72) (width 0.25) (layer "F.Cu") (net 9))
 (segment (start 57.97 62.13) (end 62.29 62.13) (width 0.25) (layer "F.Cu") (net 9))
 (segment (start 62.7 61.72) (end 62.7 61.425) (width 0.25) (layer "F.Cu") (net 9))
 (segment (start 62.0058 63.225) (end 59.5 63.225) (width 0.25) (layer "F.Cu") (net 7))
 (segment (start 59.545 63.18) (end 59.5 63.225) (width 0.25) (layer "F.Cu") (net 7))
 (segment (start 64.5202 63.981) (end 62.7618 63.981) (width 0.25) (layer "F.Cu") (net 7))
 (segment (start 62.7618 63.981) (end 62.0058 63.225) (width 0.25) (layer "F.Cu") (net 7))
 (segment (start 66.7952 67.346) (end 66.6602 67.481) (width 0.25) (layer "F.Cu") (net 6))
 (segment (start 67.7164 67.3608) (end 68.4276 67.3608) (width 0.25) (layer "F.Cu") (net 6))
 (segment (start 66.7952 65.881) (end 66.7952 67.196) (width 0.25) (layer "F.Cu") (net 6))
 (segment (start 66.5226 67.481) (end 67.5962 67.481) (width 0.25) (layer "F.Cu") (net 6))
 (segment (start 66.5226 67.481) (end 66.1702 67.481) (width 0.25) (layer "F.Cu") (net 6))
 (segment (start 66.7952 67.196) (end 66.7952 67.346) (width 0.25) (layer "F.Cu") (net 6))
 (segment (start 66.6602 67.481) (end 66.5226 67.481) (width 0.25) (layer "F.Cu") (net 6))
 (segment (start 67.5962 67.481) (end 67.7164 67.3608) (width 0.25) (layer "F.Cu") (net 6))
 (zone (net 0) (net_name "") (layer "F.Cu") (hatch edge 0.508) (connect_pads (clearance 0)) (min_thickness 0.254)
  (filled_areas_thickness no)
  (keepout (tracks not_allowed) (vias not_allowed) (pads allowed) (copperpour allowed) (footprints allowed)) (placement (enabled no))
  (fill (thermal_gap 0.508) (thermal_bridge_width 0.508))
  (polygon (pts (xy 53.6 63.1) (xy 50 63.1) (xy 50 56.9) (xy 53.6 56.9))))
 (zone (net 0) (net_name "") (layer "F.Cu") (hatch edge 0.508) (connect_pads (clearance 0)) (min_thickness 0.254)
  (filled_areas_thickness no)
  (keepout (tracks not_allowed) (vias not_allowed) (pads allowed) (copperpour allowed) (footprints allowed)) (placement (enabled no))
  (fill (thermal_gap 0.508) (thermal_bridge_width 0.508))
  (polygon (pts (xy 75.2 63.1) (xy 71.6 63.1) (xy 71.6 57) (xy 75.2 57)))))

